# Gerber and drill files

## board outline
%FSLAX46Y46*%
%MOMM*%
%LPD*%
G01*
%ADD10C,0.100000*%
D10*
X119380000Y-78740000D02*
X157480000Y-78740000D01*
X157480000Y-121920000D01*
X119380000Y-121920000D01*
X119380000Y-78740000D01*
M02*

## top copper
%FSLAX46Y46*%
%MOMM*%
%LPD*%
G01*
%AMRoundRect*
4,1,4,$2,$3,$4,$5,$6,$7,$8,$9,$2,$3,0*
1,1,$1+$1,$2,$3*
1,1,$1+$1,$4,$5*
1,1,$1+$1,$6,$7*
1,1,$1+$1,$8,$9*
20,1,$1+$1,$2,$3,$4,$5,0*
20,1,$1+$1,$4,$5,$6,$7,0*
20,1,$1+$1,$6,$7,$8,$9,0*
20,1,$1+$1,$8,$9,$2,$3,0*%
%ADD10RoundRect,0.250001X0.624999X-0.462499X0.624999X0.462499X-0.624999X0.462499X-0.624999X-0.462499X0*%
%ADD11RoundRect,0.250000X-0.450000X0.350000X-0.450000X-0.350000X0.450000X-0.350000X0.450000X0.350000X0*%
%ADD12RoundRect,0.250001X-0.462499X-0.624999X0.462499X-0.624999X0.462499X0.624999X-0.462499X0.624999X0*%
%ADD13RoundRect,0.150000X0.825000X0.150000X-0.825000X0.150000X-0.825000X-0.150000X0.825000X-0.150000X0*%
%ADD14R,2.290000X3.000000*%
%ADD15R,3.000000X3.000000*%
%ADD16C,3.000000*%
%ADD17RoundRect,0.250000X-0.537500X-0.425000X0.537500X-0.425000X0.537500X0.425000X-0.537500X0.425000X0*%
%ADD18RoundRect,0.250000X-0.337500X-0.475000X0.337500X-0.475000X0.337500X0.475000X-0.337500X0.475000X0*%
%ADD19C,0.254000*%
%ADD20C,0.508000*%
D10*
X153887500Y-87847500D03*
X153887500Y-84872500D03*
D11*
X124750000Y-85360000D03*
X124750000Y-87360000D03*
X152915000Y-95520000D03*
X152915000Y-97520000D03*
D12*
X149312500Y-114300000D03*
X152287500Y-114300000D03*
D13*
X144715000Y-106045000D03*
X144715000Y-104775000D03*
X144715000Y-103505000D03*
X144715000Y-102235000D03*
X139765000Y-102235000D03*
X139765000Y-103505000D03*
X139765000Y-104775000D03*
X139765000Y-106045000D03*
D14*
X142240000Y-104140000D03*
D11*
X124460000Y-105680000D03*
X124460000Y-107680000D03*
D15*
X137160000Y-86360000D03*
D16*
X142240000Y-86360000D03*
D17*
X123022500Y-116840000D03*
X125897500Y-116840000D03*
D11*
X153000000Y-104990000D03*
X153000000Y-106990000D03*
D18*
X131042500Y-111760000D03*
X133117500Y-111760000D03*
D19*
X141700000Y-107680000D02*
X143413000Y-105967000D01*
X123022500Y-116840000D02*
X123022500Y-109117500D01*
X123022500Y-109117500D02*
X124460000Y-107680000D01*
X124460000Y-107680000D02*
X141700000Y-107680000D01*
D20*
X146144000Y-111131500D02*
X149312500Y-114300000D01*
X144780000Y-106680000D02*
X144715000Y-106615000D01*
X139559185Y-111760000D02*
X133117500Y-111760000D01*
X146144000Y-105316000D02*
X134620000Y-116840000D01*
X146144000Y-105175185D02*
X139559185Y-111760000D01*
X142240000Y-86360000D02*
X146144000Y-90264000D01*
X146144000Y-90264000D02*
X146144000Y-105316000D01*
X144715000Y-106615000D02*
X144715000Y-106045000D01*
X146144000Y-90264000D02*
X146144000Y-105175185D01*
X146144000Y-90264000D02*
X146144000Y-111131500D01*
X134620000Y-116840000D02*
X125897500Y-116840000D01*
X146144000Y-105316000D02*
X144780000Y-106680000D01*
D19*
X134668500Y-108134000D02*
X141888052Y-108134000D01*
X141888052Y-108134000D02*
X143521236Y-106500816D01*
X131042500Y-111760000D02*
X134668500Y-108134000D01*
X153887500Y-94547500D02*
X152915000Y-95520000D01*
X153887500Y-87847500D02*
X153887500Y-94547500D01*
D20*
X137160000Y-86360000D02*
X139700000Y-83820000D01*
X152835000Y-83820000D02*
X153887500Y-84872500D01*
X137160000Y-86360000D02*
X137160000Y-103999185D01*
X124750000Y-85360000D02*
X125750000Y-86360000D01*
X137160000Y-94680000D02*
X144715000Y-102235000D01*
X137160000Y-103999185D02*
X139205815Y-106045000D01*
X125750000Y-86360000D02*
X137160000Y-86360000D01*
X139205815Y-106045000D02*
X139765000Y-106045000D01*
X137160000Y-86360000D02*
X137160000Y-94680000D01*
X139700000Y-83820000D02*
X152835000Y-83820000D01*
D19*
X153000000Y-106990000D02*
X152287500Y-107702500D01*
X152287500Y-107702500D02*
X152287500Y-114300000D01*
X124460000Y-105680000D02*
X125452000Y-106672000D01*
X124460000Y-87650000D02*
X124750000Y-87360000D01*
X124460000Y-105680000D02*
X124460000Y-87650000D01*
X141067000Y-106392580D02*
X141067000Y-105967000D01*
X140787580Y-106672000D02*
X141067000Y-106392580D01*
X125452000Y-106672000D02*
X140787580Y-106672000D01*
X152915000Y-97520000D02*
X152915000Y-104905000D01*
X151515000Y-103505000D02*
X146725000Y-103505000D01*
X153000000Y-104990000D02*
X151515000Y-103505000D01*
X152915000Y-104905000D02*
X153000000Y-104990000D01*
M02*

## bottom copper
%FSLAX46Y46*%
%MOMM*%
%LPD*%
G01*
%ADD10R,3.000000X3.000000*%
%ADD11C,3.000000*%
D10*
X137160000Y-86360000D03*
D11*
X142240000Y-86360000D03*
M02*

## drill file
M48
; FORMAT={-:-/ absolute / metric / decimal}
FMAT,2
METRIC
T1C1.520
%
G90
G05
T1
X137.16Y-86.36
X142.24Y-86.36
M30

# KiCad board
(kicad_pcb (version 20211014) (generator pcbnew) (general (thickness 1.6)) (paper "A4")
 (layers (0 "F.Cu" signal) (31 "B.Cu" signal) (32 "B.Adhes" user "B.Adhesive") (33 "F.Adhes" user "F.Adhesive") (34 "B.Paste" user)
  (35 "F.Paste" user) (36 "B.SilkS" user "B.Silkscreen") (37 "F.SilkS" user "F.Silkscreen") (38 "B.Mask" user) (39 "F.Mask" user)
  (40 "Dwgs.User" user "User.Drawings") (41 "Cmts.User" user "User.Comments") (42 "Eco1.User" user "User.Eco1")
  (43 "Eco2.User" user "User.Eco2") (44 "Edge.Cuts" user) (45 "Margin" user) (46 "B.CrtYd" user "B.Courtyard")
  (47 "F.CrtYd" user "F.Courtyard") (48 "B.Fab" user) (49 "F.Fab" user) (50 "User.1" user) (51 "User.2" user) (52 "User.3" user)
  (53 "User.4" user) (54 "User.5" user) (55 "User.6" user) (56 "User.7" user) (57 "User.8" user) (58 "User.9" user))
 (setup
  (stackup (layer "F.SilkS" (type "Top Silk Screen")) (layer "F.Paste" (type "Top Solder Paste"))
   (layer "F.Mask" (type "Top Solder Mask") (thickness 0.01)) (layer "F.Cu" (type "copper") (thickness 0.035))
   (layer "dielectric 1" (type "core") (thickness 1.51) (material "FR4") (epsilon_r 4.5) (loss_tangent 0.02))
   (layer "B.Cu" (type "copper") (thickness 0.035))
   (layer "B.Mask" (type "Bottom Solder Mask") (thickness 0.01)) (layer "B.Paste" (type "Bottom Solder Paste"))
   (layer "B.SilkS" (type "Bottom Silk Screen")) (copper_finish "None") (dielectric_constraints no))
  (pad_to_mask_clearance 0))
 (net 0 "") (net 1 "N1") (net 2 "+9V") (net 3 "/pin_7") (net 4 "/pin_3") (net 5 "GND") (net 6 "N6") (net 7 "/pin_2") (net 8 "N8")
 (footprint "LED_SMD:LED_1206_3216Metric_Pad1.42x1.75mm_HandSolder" (layer "F.Cu") (at 153.8875 86.36 90)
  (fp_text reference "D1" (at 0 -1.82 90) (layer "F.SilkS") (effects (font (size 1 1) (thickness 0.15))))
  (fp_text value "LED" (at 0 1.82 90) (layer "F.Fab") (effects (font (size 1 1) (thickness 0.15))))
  (pad "1" smd roundrect (at -1.4875 0 90) (size 1.425 1.75) (layers "F.Cu" "F.Paste" "F.Mask") (roundrect_rratio 0.175439) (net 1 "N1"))
  (pad "2" smd roundrect (at 1.4875 0 90) (size 1.425 1.75) (layers "F.Cu" "F.Paste" "F.Mask") (roundrect_rratio 0.175439) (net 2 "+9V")))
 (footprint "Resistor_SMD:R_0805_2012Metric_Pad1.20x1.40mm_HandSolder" (layer "F.Cu") (at 124.75 86.36 -90)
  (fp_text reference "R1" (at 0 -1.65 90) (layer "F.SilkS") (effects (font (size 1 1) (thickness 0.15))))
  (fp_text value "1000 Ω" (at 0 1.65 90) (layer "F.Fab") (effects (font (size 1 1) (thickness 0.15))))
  (pad "1" smd roundrect (at -1 0 270) (size 1.2 1.4) (layers "F.Cu" "F.Paste" "F.Mask") (roundrect_rratio 0.208333) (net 2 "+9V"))
  (pad "2" smd roundrect (at 1 0 270) (size 1.2 1.4) (layers "F.Cu" "F.Paste" "F.Mask") (roundrect_rratio 0.208333) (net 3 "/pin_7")))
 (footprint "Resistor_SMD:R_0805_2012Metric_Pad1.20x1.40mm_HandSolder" (layer "F.Cu") (at 152.915 96.52 -90)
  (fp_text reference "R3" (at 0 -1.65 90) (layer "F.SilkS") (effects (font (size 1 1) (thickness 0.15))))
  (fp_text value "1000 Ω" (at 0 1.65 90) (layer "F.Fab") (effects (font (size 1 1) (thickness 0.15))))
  (pad "1" smd roundrect (at -1 0 270) (size 1.2 1.4) (layers "F.Cu" "F.Paste" "F.Mask") (roundrect_rratio 0.208333) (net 1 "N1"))
  (pad "2" smd roundrect (at 1 0 270) (size 1.2 1.4) (layers "F.Cu" "F.Paste" "F.Mask") (roundrect_rratio 0.208333) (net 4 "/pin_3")))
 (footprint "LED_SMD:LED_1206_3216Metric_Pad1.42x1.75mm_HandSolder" (layer "F.Cu") (at 150.8 114.3)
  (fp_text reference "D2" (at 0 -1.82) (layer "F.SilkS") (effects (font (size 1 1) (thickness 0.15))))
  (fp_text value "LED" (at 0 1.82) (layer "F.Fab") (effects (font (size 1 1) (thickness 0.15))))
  (pad "1" smd roundrect (at -1.4875 0) (size 1.425 1.75) (layers "F.Cu" "F.Paste" "F.Mask") (roundrect_rratio 0.175439) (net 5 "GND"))
  (pad "2" smd roundrect (at 1.4875 0) (size 1.425 1.75) (layers "F.Cu" "F.Paste" "F.Mask") (roundrect_rratio 0.175439) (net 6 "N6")))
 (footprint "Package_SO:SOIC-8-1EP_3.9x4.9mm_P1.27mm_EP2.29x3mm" (layer "F.Cu") (at 142.24 104.14 180)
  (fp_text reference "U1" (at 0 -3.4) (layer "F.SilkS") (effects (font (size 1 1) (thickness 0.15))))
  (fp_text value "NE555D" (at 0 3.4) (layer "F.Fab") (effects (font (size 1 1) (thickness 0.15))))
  (pad "" smd roundrect (at 0.57 0.75 180) (size 0.92 1.21) (layers "F.Paste") (roundrect_rratio 0.25))
  (pad "" smd roundrect (at -0.57 0.75 180) (size 0.92 1.21) (layers "F.Paste") (roundrect_rratio 0.25))
  (pad "" smd roundrect (at 0.57 -0.75 180) (size 0.92 1.21) (layers "F.Paste") (roundrect_rratio 0.25))
  (pad "" smd roundrect (at -0.57 -0.75 180) (size 0.92 1.21) (layers "F.Paste") (roundrect_rratio 0.25))
  (pad "1" smd roundrect (at -2.475 -1.905 180) (size 1.95 0.6) (layers "F.Cu" "F.Paste" "F.Mask") (roundrect_rratio 0.25) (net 5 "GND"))
  (pad "2" smd roundrect (at -2.475 -0.635 180) (size 1.95 0.6) (layers "F.Cu" "F.Paste" "F.Mask") (roundrect_rratio 0.25) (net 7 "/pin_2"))
  (pad "3" smd roundrect (at -2.475 0.635 180) (size 1.95 0.6) (layers "F.Cu" "F.Paste" "F.Mask") (roundrect_rratio 0.25) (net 4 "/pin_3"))
  (pad "4" smd roundrect (at -2.475 1.905 180) (size 1.95 0.6) (layers "F.Cu" "F.Paste" "F.Mask") (roundrect_rratio 0.25) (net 2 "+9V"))
  (pad "5" smd roundrect (at 2.475 1.905 180) (size 1.95 0.6) (layers "F.Cu" "F.Paste" "F.Mask") (roundrect_rratio 0.25) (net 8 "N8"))
  (pad "6" smd roundrect (at 2.475 0.635 180) (size 1.95 0.6) (layers "F.Cu" "F.Paste" "F.Mask") (roundrect_rratio 0.25) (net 7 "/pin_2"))
  (pad "7" smd roundrect (at 2.475 -0.635 180) (size 1.95 0.6) (layers "F.Cu" "F.Paste" "F.Mask") (roundrect_rratio 0.25) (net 3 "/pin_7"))
  (pad "8" smd roundrect (at 2.475 -1.905 180) (size 1.95 0.6) (layers "F.Cu" "F.Paste" "F.Mask") (roundrect_rratio 0.25) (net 2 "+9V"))
  (pad "9" smd rect (at 0 0 180) (size 2.29 3) (layers "F.Cu" "F.Mask")))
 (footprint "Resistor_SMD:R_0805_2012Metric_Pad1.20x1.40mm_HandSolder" (layer "F.Cu") (at 124.46 106.68 -90)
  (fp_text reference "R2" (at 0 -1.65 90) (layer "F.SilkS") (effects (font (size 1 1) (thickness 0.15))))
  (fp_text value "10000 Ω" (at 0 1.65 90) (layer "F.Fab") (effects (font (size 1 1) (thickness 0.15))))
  (pad "1" smd roundrect (at -1 0 270) (size 1.2 1.4) (layers "F.Cu" "F.Paste" "F.Mask") (roundrect_rratio 0.208333) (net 3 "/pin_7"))
  (pad "2" smd roundrect (at 1 0 270) (size 1.2 1.4) (layers "F.Cu" "F.Paste" "F.Mask") (roundrect_rratio 0.208333) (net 7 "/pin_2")))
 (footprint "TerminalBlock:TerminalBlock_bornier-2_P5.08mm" (layer "F.Cu") (at 137.16 86.36)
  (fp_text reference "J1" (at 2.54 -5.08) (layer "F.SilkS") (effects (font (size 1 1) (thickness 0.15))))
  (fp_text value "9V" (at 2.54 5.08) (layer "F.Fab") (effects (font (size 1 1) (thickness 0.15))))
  (pad "1" thru_hole rect (at 0 0) (size 3 3) (drill 1.52) (layers *.Cu *.Mask) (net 2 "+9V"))
  (pad "2" thru_hole circle (at 5.08 0) (size 3 3) (drill 1.52) (layers *.Cu *.Mask) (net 5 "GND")))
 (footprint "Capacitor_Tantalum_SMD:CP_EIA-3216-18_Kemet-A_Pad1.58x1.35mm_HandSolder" (layer "F.Cu") (at 124.46 116.84)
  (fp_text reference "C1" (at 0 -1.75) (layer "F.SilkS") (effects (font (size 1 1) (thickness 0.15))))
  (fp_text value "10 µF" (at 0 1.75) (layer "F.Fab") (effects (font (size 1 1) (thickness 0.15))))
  (pad "1" smd roundrect (at -1.4375 0) (size 1.575 1.35) (layers "F.Cu" "F.Paste" "F.Mask") (roundrect_rratio 0.185185) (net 7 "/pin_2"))
  (pad "2" smd roundrect (at 1.4375 0) (size 1.575 1.35) (layers "F.Cu" "F.Paste" "F.Mask") (roundrect_rratio 0.185185) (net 5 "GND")))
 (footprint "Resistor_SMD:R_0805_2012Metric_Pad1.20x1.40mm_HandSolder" (layer "F.Cu") (at 153 105.99 -90)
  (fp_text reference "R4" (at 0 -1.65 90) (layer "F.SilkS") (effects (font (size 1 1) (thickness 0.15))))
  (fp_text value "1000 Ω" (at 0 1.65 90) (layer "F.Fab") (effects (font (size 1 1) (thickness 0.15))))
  (pad "1" smd roundrect (at -1 0 270) (size 1.2 1.4) (layers "F.Cu" "F.Paste" "F.Mask") (roundrect_rratio 0.208333) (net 4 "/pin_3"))
  (pad "2" smd roundrect (at 1 0 270) (size 1.2 1.4) (layers "F.Cu" "F.Paste" "F.Mask") (roundrect_rratio 0.208333) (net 6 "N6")))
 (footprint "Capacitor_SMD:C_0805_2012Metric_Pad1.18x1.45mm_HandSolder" (layer "F.Cu") (at 132.08 111.76)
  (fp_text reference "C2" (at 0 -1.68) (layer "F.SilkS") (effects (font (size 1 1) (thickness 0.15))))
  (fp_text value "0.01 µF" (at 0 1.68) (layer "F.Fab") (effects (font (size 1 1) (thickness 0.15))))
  (pad "1" smd roundrect (at -1.0375 0) (size 1.175 1.45) (layers "F.Cu" "F.Paste" "F.Mask") (roundrect_rratio 0.212766) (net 8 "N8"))
  (pad "2" smd roundrect (at 1.0375 0) (size 1.175 1.45) (layers "F.Cu" "F.Paste" "F.Mask") (roundrect_rratio 0.212766) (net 5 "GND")))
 (gr_rect (start 119.38 78.74) (end 157.48 121.92) (layer "Edge.Cuts") (width 0.1) (fill none))
 (segment (start 141.7 107.68) (end 143.413 105.967) (width 0.254) (layer "F.Cu") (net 7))
 (segment (start 123.0225 116.84) (end 123.0225 109.1175) (width 0.254) (layer "F.Cu") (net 7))
 (segment (start 123.0225 109.1175) (end 124.46 107.68) (width 0.254) (layer "F.Cu") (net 7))
 (segment (start 124.46 107.68) (end 141.7 107.68) (width 0.254) (layer "F.Cu") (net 7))
 (segment (start 146.144 111.1315) (end 149.3125 114.3) (width 0.508) (layer "F.Cu") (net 5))
 (segment (start 144.78 106.68) (end 144.715 106.615) (width 0.508) (layer "F.Cu") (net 5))
 (segment (start 139.559185 111.76) (end 133.1175 111.76) (width 0.508) (layer "F.Cu") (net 5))
 (segment (start 146.144 105.316) (end 134.62 116.84) (width 0.508) (layer "F.Cu") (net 5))
 (segment (start 146.144 105.175185) (end 139.559185 111.76) (width 0.508) (layer "F.Cu") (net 5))
 (segment (start 142.24 86.36) (end 146.144 90.264) (width 0.508) (layer "F.Cu") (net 5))
 (segment (start 146.144 90.264) (end 146.144 105.316) (width 0.508) (layer "F.Cu") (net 5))
 (segment (start 144.715 106.615) (end 144.715 106.045) (width 0.508) (layer "F.Cu") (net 5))
 (segment (start 146.144 90.264) (end 146.144 105.175185) (width 0.508) (layer "F.Cu") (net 5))
 (segment (start 146.144 90.264) (end 146.144 111.1315) (width 0.508) (layer "F.Cu") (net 5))
 (segment (start 134.62 116.84) (end 125.8975 116.84) (width 0.508) (layer "F.Cu") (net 5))
 (segment (start 146.144 105.316) (end 144.78 106.68) (width 0.508) (layer "F.Cu") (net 5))
 (segment (start 134.6685 108.134) (end 141.888052 108.134) (width 0.254) (layer "F.Cu") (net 8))
 (segment (start 141.888052 108.134) (end 143.521236 106.500816) (width 0.254) (layer "F.Cu") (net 8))
 (segment (start 131.0425 111.76) (end 134.6685 108.134) (width 0.254) (layer "F.Cu") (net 8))
 (segment (start 153.8875 94.5475) (end 152.915 95.52) (width 0.254) (layer "F.Cu") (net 1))
 (segment (start 153.8875 87.8475) (end 153.8875 94.5475) (width 0.254) (layer "F.Cu") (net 1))
 (segment (start 137.16 86.36) (end 139.7 83.82) (width 0.508) (layer "F.Cu") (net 2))
 (segment (start 152.835 83.82) (end 153.8875 84.8725) (width 0.508) (layer "F.Cu") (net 2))
 (segment (start 137.16 86.36) (end 137.16 103.999185) (width 0.508) (layer "F.Cu") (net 2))
 (segment (start 124.75 85.36) (end 125.75 86.36) (width 0.508) (layer "F.Cu") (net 2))
 (segment (start 137.16 94.68) (end 144.715 102.235) (width 0.508) (layer "F.Cu") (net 2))
 (segment (start 137.16 103.999185) (end 139.205815 106.045) (width 0.508) (layer "F.Cu") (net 2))
 (segment (start 125.75 86.36) (end 137.16 86.36) (width 0.508) (layer "F.Cu") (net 2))
 (segment (start 139.205815 106.045) (end 139.765 106.045) (width 0.508) (layer "F.Cu") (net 2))
 (segment (start 137.16 86.36) (end 137.16 94.68) (width 0.508) (layer "F.Cu") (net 2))
 (segment (start 139.7 83.82) (end 152.835 83.82) (width 0.508) (layer "F.Cu") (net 2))
 (segment (start 153 106.99) (end 152.2875 107.7025) (width 0.254) (layer "F.Cu") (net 6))
 (segment (start 152.2875 107.7025) (end 152.2875 114.3) (width 0.254) (layer "F.Cu") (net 6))
 (segment (start 124.46 105.68) (end 125.452 106.672) (width 0.254) (layer "F.Cu") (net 3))
 (segment (start 124.46 87.65) (end 124.75 87.36) (width 0.254) (layer "F.Cu") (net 3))
 (segment (start 124.46 105.68) (end 124.46 87.65) (width 0.254) (layer "F.Cu") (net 3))
 (segment (start 141.067 106.39258) (end 141.067 105.967) (width 0.254) (layer "F.Cu") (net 3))
 (segment (start 140.78758 106.672) (end 141.067 106.39258) (width 0.254) (layer "F.Cu") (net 3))
 (segment (start 125.452 106.672) (end 140.78758 106.672) (width 0.254) (layer "F.Cu") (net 3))
 (segment (start 152.915 97.52) (end 152.915 104.905) (width 0.254) (layer "F.Cu") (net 4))
 (segment (start 151.515 103.505) (end 146.725 103.505) (width 0.254) (layer "F.Cu") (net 4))
 (segment (start 153 104.99) (end 151.515 103.505) (width 0.254) (layer "F.Cu") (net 4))
 (segment (start 152.915 104.905) (end 153 104.99) (width 0.254) (layer "F.Cu") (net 4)))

